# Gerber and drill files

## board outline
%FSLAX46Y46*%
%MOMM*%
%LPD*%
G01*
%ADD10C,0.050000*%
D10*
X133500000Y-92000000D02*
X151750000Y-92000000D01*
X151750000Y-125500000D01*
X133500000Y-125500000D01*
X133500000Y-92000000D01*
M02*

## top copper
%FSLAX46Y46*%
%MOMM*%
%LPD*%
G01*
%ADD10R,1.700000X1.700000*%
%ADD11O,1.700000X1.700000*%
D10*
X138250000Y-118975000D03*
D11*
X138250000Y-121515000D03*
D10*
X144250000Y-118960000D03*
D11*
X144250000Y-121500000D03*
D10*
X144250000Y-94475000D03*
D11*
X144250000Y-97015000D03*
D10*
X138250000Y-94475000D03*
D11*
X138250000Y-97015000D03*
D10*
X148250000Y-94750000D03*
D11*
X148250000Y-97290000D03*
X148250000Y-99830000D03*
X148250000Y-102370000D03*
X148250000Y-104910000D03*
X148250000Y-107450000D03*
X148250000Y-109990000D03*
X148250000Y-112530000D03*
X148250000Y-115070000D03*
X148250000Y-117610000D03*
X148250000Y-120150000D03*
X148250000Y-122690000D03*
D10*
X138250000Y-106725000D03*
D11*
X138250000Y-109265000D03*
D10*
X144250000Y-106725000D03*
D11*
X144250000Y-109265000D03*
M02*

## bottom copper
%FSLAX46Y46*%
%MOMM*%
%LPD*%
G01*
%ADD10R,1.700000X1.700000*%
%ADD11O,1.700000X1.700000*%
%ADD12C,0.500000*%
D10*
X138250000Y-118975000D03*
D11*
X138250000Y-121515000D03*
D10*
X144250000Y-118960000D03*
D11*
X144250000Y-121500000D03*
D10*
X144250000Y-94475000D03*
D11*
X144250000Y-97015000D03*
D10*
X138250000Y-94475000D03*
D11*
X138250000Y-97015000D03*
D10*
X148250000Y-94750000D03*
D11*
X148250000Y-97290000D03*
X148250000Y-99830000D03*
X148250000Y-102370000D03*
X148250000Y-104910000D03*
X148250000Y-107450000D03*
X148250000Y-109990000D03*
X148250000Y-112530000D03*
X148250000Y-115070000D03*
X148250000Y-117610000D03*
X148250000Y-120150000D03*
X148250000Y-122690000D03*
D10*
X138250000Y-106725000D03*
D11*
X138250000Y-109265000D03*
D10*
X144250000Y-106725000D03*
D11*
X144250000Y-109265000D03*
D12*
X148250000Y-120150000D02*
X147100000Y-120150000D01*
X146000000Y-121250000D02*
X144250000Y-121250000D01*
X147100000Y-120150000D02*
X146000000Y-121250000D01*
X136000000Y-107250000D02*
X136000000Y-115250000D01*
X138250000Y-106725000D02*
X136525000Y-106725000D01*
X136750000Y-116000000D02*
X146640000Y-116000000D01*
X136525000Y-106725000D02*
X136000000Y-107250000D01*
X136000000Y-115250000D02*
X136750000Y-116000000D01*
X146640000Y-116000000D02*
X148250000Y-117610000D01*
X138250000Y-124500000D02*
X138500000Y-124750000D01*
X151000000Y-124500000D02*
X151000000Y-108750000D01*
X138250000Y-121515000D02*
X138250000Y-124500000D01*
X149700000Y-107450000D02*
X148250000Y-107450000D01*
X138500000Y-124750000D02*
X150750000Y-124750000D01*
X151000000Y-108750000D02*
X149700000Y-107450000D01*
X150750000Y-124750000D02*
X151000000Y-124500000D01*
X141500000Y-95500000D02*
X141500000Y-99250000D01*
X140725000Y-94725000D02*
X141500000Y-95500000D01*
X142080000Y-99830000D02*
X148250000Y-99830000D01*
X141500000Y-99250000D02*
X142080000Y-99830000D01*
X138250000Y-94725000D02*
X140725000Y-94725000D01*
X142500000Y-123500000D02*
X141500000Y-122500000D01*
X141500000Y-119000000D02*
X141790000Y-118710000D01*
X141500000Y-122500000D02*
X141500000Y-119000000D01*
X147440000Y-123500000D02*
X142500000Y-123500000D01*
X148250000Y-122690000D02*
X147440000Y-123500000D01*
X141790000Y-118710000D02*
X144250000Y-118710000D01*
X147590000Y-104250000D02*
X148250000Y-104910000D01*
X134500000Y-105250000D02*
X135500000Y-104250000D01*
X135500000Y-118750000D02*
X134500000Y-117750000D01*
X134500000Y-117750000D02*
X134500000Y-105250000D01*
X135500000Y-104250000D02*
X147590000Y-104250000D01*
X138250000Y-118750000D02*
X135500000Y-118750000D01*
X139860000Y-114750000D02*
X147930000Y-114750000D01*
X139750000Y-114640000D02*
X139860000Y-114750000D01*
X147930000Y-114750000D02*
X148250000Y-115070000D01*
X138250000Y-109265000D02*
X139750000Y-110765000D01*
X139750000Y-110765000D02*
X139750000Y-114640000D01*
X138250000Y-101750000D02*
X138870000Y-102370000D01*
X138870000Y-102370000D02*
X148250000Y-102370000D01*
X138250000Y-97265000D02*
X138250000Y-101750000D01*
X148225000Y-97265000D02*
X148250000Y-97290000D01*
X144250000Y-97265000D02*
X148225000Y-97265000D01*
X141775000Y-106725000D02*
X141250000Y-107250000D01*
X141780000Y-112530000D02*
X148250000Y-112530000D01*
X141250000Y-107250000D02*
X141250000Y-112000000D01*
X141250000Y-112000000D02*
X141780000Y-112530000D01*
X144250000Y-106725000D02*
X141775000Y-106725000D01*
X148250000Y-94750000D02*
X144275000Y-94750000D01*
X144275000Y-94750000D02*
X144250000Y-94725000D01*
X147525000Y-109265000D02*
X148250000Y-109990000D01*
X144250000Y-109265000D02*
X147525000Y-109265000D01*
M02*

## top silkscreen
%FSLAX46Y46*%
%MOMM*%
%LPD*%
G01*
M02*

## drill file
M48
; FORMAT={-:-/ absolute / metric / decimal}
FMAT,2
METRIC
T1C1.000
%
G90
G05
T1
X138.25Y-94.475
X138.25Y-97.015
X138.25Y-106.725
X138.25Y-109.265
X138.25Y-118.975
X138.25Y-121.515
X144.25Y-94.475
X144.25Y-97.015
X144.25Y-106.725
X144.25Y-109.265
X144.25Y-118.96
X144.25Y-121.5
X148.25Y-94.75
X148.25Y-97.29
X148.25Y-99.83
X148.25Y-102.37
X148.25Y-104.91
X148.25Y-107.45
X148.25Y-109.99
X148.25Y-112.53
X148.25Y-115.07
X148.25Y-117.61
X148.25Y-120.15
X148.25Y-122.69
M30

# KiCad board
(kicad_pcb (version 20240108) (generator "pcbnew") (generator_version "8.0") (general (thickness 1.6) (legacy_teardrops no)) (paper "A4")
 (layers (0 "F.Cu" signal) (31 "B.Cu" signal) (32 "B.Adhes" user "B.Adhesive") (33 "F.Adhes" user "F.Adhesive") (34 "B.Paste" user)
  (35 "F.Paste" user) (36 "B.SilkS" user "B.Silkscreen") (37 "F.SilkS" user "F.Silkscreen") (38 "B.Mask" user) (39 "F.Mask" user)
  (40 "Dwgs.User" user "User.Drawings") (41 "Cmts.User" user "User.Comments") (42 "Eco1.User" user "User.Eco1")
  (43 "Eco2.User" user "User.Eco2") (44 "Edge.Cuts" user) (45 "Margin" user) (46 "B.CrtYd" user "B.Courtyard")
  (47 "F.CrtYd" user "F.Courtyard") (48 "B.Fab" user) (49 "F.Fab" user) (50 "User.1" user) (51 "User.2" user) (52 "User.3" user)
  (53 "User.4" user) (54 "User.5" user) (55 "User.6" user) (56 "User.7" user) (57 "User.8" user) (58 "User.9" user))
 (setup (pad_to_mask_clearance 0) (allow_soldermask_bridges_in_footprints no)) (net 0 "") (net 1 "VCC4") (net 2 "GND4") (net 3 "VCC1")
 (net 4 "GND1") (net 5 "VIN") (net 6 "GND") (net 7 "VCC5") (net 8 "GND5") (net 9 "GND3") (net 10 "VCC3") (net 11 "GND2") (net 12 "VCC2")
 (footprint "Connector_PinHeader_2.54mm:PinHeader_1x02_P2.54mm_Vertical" (layer "B.Cu") (at 138.25 118.975 180)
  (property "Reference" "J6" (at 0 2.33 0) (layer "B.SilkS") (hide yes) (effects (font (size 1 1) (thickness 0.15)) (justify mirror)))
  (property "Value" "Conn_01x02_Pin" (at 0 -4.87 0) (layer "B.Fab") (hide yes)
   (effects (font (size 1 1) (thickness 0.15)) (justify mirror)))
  (pad "1" thru_hole rect (at 0 0 180) (size 1.7 1.7) (drill 1) (layers "*.Cu" "*.Mask") (remove_unused_layers no) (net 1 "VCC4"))
  (pad "2" thru_hole oval (at 0 -2.54 180) (size 1.7 1.7) (drill 1) (layers "*.Cu" "*.Mask") (remove_unused_layers no) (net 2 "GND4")))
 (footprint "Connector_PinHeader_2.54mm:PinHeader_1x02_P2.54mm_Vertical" (layer "B.Cu") (at 144.25 118.96 180)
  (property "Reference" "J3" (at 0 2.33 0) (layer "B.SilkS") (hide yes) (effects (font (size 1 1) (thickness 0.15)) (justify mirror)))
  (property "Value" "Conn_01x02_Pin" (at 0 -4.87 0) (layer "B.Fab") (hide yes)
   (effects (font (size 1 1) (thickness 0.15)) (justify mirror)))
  (pad "1" thru_hole rect (at 0 0 180) (size 1.7 1.7) (drill 1) (layers "*.Cu" "*.Mask") (remove_unused_layers no) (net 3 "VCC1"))
  (pad "2" thru_hole oval (at 0 -2.54 180) (size 1.7 1.7) (drill 1) (layers "*.Cu" "*.Mask") (remove_unused_layers no) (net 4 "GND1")))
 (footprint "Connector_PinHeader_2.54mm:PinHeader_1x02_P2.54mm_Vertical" (layer "B.Cu") (at 144.25 94.475 180)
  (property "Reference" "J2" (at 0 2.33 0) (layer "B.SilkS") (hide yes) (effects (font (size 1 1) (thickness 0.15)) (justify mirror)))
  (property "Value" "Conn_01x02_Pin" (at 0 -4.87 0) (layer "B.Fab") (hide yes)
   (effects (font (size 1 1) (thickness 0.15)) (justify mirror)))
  (pad "1" thru_hole rect (at 0 0 180) (size 1.7 1.7) (drill 1) (layers "*.Cu" "*.Mask") (remove_unused_layers no) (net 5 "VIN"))
  (pad "2" thru_hole oval (at 0 -2.54 180) (size 1.7 1.7) (drill 1) (layers "*.Cu" "*.Mask") (remove_unused_layers no) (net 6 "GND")))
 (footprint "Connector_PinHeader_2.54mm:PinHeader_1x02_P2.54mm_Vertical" (layer "B.Cu") (at 138.25 94.475 180)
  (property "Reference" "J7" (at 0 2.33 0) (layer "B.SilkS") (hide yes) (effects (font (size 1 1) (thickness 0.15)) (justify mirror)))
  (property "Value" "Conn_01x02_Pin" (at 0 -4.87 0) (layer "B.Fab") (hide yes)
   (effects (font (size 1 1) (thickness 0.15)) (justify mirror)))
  (pad "1" thru_hole rect (at 0 0 180) (size 1.7 1.7) (drill 1) (layers "*.Cu" "*.Mask") (remove_unused_layers no) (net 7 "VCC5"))
  (pad "2" thru_hole oval (at 0 -2.54 180) (size 1.7 1.7) (drill 1) (layers "*.Cu" "*.Mask") (remove_unused_layers no) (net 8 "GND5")))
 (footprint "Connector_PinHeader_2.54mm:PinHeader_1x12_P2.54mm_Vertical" (layer "B.Cu") (at 148.25 94.75 180)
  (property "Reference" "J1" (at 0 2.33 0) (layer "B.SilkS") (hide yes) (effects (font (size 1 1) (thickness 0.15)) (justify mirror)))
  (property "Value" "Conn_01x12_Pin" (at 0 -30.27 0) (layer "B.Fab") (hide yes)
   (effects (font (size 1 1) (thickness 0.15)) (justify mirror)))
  (pad "1" thru_hole rect (at 0 0 180) (size 1.7 1.7) (drill 1) (layers "*.Cu" "*.Mask") (remove_unused_layers no) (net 5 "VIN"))
  (pad "2" thru_hole oval (at 0 -2.54 180) (size 1.7 1.7) (drill 1) (layers "*.Cu" "*.Mask") (remove_unused_layers no) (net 6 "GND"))
  (pad "3" thru_hole oval (at 0 -5.08 180) (size 1.7 1.7) (drill 1) (layers "*.Cu" "*.Mask") (remove_unused_layers no) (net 7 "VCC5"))
  (pad "4" thru_hole oval (at 0 -7.62 180) (size 1.7 1.7) (drill 1) (layers "*.Cu" "*.Mask") (remove_unused_layers no) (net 8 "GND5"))
  (pad "5" thru_hole oval (at 0 -10.16 180) (size 1.7 1.7) (drill 1) (layers "*.Cu" "*.Mask") (remove_unused_layers no) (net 1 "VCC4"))
  (pad "6" thru_hole oval (at 0 -12.7 180) (size 1.7 1.7) (drill 1) (layers "*.Cu" "*.Mask") (remove_unused_layers no) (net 2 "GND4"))
  (pad "7" thru_hole oval (at 0 -15.24 180) (size 1.7 1.7) (drill 1) (layers "*.Cu" "*.Mask") (remove_unused_layers no) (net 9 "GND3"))
  (pad "8" thru_hole oval (at 0 -17.78 180) (size 1.7 1.7) (drill 1) (layers "*.Cu" "*.Mask") (remove_unused_layers no) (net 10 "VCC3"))
  (pad "9" thru_hole oval (at 0 -20.32 180) (size 1.7 1.7) (drill 1) (layers "*.Cu" "*.Mask") (remove_unused_layers no) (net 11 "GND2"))
  (pad "10" thru_hole oval (at 0 -22.86 180) (size 1.7 1.7) (drill 1) (layers "*.Cu" "*.Mask") (remove_unused_layers no) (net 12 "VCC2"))
  (pad "11" thru_hole oval (at 0 -25.4 180) (size 1.7 1.7) (drill 1) (layers "*.Cu" "*.Mask") (remove_unused_layers no) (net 4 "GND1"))
  (pad "12" thru_hole oval (at 0 -27.94 180) (size 1.7 1.7) (drill 1) (layers "*.Cu" "*.Mask") (remove_unused_layers no) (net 3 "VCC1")))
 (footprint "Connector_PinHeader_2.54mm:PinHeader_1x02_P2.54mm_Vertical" (layer "B.Cu") (at 138.25 106.725 180)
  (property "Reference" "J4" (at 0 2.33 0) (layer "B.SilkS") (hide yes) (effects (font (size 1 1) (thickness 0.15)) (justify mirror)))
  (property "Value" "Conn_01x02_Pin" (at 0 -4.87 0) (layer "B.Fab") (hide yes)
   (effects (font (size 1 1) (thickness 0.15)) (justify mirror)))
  (pad "1" thru_hole rect (at 0 0 180) (size 1.7 1.7) (drill 1) (layers "*.Cu" "*.Mask") (remove_unused_layers no) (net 12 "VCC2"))
  (pad "2" thru_hole oval (at 0 -2.54 180) (size 1.7 1.7) (drill 1) (layers "*.Cu" "*.Mask") (remove_unused_layers no) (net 11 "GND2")))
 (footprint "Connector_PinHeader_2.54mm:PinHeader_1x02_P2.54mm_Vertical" (layer "B.Cu") (at 144.25 106.725 180)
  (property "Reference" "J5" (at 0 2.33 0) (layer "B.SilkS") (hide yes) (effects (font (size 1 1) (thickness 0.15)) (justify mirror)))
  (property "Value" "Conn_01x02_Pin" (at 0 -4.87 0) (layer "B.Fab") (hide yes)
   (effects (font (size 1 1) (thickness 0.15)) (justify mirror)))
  (pad "1" thru_hole rect (at 0 0 180) (size 1.7 1.7) (drill 1) (layers "*.Cu" "*.Mask") (remove_unused_layers no) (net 10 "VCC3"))
  (pad "2" thru_hole oval (at 0 -2.54 180) (size 1.7 1.7) (drill 1) (layers "*.Cu" "*.Mask") (remove_unused_layers no) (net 9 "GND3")))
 (gr_rect (start 133.5 92) (end 151.75 125.5) (stroke (width 0.05) (type default)) (fill none) (layer "Edge.Cuts"))
 (segment (start 148.25 120.15) (end 147.1 120.15) (width 0.5) (layer "B.Cu") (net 4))
 (segment (start 146 121.25) (end 144.25 121.25) (width 0.5) (layer "B.Cu") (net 4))
 (segment (start 147.1 120.15) (end 146 121.25) (width 0.5) (layer "B.Cu") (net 4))
 (segment (start 136 107.25) (end 136 115.25) (width 0.5) (layer "B.Cu") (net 12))
 (segment (start 138.25 106.725) (end 136.525 106.725) (width 0.5) (layer "B.Cu") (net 12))
 (segment (start 136.75 116) (end 146.64 116) (width 0.5) (layer "B.Cu") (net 12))
 (segment (start 136.525 106.725) (end 136 107.25) (width 0.5) (layer "B.Cu") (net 12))
 (segment (start 136 115.25) (end 136.75 116) (width 0.5) (layer "B.Cu") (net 12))
 (segment (start 146.64 116) (end 148.25 117.61) (width 0.5) (layer "B.Cu") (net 12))
 (segment (start 138.25 124.5) (end 138.5 124.75) (width 0.5) (layer "B.Cu") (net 2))
 (segment (start 151 124.5) (end 151 108.75) (width 0.5) (layer "B.Cu") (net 2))
 (segment (start 138.25 121.515) (end 138.25 124.5) (width 0.5) (layer "B.Cu") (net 2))
 (segment (start 149.7 107.45) (end 148.25 107.45) (width 0.5) (layer "B.Cu") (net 2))
 (segment (start 138.5 124.75) (end 150.75 124.75) (width 0.5) (layer "B.Cu") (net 2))
 (segment (start 151 108.75) (end 149.7 107.45) (width 0.5) (layer "B.Cu") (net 2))
 (segment (start 150.75 124.75) (end 151 124.5) (width 0.5) (layer "B.Cu") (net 2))
 (segment (start 141.5 95.5) (end 141.5 99.25) (width 0.5) (layer "B.Cu") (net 7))
 (segment (start 140.725 94.725) (end 141.5 95.5) (width 0.5) (layer "B.Cu") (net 7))
 (segment (start 142.08 99.83) (end 148.25 99.83) (width 0.5) (layer "B.Cu") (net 7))
 (segment (start 141.5 99.25) (end 142.08 99.83) (width 0.5) (layer "B.Cu") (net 7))
 (segment (start 138.25 94.725) (end 140.725 94.725) (width 0.5) (layer "B.Cu") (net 7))
 (segment (start 142.5 123.5) (end 141.5 122.5) (width 0.5) (layer "B.Cu") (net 3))
 (segment (start 141.5 119) (end 141.79 118.71) (width 0.5) (layer "B.Cu") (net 3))
 (segment (start 141.5 122.5) (end 141.5 119) (width 0.5) (layer "B.Cu") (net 3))
 (segment (start 147.44 123.5) (end 142.5 123.5) (width 0.5) (layer "B.Cu") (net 3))
 (segment (start 148.25 122.69) (end 147.44 123.5) (width 0.5) (layer "B.Cu") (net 3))
 (segment (start 141.79 118.71) (end 144.25 118.71) (width 0.5) (layer "B.Cu") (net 3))
 (segment (start 147.59 104.25) (end 148.25 104.91) (width 0.5) (layer "B.Cu") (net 1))
 (segment (start 134.5 105.25) (end 135.5 104.25) (width 0.5) (layer "B.Cu") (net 1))
 (segment (start 135.5 118.75) (end 134.5 117.75) (width 0.5) (layer "B.Cu") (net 1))
 (segment (start 134.5 117.75) (end 134.5 105.25) (width 0.5) (layer "B.Cu") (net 1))
 (segment (start 135.5 104.25) (end 147.59 104.25) (width 0.5) (layer "B.Cu") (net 1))
 (segment (start 138.25 118.75) (end 135.5 118.75) (width 0.5) (layer "B.Cu") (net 1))
 (segment (start 139.86 114.75) (end 147.93 114.75) (width 0.5) (layer "B.Cu") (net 11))
 (segment (start 139.75 114.64) (end 139.86 114.75) (width 0.5) (layer "B.Cu") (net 11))
 (segment (start 147.93 114.75) (end 148.25 115.07) (width 0.5) (layer "B.Cu") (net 11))
 (segment (start 138.25 109.265) (end 139.75 110.765) (width 0.5) (layer "B.Cu") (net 11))
 (segment (start 139.75 110.765) (end 139.75 114.64) (width 0.5) (layer "B.Cu") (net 11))
 (segment (start 138.25 101.75) (end 138.87 102.37) (width 0.5) (layer "B.Cu") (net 8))
 (segment (start 138.87 102.37) (end 148.25 102.37) (width 0.5) (layer "B.Cu") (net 8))
 (segment (start 138.25 97.265) (end 138.25 101.75) (width 0.5) (layer "B.Cu") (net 8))
 (segment (start 148.225 97.265) (end 148.25 97.29) (width 0.5) (layer "B.Cu") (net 6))
 (segment (start 144.25 97.265) (end 148.225 97.265) (width 0.5) (layer "B.Cu") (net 6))
 (segment (start 141.775 106.725) (end 141.25 107.25) (width 0.5) (layer "B.Cu") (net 10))
 (segment (start 141.78 112.53) (end 148.25 112.53) (width 0.5) (layer "B.Cu") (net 10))
 (segment (start 141.25 107.25) (end 141.25 112) (width 0.5) (layer "B.Cu") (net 10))
 (segment (start 141.25 112) (end 141.78 112.53) (width 0.5) (layer "B.Cu") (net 10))
 (segment (start 144.25 106.725) (end 141.775 106.725) (width 0.5) (layer "B.Cu") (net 10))
 (segment (start 148.25 94.75) (end 144.275 94.75) (width 0.5) (layer "B.Cu") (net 5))
 (segment (start 144.275 94.75) (end 144.25 94.725) (width 0.5) (layer "B.Cu") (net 5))
 (segment (start 147.525 109.265) (end 148.25 109.99) (width 0.5) (layer "B.Cu") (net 9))
 (segment (start 144.25 109.265) (end 147.525 109.265) (width 0.5) (layer "B.Cu") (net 9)))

